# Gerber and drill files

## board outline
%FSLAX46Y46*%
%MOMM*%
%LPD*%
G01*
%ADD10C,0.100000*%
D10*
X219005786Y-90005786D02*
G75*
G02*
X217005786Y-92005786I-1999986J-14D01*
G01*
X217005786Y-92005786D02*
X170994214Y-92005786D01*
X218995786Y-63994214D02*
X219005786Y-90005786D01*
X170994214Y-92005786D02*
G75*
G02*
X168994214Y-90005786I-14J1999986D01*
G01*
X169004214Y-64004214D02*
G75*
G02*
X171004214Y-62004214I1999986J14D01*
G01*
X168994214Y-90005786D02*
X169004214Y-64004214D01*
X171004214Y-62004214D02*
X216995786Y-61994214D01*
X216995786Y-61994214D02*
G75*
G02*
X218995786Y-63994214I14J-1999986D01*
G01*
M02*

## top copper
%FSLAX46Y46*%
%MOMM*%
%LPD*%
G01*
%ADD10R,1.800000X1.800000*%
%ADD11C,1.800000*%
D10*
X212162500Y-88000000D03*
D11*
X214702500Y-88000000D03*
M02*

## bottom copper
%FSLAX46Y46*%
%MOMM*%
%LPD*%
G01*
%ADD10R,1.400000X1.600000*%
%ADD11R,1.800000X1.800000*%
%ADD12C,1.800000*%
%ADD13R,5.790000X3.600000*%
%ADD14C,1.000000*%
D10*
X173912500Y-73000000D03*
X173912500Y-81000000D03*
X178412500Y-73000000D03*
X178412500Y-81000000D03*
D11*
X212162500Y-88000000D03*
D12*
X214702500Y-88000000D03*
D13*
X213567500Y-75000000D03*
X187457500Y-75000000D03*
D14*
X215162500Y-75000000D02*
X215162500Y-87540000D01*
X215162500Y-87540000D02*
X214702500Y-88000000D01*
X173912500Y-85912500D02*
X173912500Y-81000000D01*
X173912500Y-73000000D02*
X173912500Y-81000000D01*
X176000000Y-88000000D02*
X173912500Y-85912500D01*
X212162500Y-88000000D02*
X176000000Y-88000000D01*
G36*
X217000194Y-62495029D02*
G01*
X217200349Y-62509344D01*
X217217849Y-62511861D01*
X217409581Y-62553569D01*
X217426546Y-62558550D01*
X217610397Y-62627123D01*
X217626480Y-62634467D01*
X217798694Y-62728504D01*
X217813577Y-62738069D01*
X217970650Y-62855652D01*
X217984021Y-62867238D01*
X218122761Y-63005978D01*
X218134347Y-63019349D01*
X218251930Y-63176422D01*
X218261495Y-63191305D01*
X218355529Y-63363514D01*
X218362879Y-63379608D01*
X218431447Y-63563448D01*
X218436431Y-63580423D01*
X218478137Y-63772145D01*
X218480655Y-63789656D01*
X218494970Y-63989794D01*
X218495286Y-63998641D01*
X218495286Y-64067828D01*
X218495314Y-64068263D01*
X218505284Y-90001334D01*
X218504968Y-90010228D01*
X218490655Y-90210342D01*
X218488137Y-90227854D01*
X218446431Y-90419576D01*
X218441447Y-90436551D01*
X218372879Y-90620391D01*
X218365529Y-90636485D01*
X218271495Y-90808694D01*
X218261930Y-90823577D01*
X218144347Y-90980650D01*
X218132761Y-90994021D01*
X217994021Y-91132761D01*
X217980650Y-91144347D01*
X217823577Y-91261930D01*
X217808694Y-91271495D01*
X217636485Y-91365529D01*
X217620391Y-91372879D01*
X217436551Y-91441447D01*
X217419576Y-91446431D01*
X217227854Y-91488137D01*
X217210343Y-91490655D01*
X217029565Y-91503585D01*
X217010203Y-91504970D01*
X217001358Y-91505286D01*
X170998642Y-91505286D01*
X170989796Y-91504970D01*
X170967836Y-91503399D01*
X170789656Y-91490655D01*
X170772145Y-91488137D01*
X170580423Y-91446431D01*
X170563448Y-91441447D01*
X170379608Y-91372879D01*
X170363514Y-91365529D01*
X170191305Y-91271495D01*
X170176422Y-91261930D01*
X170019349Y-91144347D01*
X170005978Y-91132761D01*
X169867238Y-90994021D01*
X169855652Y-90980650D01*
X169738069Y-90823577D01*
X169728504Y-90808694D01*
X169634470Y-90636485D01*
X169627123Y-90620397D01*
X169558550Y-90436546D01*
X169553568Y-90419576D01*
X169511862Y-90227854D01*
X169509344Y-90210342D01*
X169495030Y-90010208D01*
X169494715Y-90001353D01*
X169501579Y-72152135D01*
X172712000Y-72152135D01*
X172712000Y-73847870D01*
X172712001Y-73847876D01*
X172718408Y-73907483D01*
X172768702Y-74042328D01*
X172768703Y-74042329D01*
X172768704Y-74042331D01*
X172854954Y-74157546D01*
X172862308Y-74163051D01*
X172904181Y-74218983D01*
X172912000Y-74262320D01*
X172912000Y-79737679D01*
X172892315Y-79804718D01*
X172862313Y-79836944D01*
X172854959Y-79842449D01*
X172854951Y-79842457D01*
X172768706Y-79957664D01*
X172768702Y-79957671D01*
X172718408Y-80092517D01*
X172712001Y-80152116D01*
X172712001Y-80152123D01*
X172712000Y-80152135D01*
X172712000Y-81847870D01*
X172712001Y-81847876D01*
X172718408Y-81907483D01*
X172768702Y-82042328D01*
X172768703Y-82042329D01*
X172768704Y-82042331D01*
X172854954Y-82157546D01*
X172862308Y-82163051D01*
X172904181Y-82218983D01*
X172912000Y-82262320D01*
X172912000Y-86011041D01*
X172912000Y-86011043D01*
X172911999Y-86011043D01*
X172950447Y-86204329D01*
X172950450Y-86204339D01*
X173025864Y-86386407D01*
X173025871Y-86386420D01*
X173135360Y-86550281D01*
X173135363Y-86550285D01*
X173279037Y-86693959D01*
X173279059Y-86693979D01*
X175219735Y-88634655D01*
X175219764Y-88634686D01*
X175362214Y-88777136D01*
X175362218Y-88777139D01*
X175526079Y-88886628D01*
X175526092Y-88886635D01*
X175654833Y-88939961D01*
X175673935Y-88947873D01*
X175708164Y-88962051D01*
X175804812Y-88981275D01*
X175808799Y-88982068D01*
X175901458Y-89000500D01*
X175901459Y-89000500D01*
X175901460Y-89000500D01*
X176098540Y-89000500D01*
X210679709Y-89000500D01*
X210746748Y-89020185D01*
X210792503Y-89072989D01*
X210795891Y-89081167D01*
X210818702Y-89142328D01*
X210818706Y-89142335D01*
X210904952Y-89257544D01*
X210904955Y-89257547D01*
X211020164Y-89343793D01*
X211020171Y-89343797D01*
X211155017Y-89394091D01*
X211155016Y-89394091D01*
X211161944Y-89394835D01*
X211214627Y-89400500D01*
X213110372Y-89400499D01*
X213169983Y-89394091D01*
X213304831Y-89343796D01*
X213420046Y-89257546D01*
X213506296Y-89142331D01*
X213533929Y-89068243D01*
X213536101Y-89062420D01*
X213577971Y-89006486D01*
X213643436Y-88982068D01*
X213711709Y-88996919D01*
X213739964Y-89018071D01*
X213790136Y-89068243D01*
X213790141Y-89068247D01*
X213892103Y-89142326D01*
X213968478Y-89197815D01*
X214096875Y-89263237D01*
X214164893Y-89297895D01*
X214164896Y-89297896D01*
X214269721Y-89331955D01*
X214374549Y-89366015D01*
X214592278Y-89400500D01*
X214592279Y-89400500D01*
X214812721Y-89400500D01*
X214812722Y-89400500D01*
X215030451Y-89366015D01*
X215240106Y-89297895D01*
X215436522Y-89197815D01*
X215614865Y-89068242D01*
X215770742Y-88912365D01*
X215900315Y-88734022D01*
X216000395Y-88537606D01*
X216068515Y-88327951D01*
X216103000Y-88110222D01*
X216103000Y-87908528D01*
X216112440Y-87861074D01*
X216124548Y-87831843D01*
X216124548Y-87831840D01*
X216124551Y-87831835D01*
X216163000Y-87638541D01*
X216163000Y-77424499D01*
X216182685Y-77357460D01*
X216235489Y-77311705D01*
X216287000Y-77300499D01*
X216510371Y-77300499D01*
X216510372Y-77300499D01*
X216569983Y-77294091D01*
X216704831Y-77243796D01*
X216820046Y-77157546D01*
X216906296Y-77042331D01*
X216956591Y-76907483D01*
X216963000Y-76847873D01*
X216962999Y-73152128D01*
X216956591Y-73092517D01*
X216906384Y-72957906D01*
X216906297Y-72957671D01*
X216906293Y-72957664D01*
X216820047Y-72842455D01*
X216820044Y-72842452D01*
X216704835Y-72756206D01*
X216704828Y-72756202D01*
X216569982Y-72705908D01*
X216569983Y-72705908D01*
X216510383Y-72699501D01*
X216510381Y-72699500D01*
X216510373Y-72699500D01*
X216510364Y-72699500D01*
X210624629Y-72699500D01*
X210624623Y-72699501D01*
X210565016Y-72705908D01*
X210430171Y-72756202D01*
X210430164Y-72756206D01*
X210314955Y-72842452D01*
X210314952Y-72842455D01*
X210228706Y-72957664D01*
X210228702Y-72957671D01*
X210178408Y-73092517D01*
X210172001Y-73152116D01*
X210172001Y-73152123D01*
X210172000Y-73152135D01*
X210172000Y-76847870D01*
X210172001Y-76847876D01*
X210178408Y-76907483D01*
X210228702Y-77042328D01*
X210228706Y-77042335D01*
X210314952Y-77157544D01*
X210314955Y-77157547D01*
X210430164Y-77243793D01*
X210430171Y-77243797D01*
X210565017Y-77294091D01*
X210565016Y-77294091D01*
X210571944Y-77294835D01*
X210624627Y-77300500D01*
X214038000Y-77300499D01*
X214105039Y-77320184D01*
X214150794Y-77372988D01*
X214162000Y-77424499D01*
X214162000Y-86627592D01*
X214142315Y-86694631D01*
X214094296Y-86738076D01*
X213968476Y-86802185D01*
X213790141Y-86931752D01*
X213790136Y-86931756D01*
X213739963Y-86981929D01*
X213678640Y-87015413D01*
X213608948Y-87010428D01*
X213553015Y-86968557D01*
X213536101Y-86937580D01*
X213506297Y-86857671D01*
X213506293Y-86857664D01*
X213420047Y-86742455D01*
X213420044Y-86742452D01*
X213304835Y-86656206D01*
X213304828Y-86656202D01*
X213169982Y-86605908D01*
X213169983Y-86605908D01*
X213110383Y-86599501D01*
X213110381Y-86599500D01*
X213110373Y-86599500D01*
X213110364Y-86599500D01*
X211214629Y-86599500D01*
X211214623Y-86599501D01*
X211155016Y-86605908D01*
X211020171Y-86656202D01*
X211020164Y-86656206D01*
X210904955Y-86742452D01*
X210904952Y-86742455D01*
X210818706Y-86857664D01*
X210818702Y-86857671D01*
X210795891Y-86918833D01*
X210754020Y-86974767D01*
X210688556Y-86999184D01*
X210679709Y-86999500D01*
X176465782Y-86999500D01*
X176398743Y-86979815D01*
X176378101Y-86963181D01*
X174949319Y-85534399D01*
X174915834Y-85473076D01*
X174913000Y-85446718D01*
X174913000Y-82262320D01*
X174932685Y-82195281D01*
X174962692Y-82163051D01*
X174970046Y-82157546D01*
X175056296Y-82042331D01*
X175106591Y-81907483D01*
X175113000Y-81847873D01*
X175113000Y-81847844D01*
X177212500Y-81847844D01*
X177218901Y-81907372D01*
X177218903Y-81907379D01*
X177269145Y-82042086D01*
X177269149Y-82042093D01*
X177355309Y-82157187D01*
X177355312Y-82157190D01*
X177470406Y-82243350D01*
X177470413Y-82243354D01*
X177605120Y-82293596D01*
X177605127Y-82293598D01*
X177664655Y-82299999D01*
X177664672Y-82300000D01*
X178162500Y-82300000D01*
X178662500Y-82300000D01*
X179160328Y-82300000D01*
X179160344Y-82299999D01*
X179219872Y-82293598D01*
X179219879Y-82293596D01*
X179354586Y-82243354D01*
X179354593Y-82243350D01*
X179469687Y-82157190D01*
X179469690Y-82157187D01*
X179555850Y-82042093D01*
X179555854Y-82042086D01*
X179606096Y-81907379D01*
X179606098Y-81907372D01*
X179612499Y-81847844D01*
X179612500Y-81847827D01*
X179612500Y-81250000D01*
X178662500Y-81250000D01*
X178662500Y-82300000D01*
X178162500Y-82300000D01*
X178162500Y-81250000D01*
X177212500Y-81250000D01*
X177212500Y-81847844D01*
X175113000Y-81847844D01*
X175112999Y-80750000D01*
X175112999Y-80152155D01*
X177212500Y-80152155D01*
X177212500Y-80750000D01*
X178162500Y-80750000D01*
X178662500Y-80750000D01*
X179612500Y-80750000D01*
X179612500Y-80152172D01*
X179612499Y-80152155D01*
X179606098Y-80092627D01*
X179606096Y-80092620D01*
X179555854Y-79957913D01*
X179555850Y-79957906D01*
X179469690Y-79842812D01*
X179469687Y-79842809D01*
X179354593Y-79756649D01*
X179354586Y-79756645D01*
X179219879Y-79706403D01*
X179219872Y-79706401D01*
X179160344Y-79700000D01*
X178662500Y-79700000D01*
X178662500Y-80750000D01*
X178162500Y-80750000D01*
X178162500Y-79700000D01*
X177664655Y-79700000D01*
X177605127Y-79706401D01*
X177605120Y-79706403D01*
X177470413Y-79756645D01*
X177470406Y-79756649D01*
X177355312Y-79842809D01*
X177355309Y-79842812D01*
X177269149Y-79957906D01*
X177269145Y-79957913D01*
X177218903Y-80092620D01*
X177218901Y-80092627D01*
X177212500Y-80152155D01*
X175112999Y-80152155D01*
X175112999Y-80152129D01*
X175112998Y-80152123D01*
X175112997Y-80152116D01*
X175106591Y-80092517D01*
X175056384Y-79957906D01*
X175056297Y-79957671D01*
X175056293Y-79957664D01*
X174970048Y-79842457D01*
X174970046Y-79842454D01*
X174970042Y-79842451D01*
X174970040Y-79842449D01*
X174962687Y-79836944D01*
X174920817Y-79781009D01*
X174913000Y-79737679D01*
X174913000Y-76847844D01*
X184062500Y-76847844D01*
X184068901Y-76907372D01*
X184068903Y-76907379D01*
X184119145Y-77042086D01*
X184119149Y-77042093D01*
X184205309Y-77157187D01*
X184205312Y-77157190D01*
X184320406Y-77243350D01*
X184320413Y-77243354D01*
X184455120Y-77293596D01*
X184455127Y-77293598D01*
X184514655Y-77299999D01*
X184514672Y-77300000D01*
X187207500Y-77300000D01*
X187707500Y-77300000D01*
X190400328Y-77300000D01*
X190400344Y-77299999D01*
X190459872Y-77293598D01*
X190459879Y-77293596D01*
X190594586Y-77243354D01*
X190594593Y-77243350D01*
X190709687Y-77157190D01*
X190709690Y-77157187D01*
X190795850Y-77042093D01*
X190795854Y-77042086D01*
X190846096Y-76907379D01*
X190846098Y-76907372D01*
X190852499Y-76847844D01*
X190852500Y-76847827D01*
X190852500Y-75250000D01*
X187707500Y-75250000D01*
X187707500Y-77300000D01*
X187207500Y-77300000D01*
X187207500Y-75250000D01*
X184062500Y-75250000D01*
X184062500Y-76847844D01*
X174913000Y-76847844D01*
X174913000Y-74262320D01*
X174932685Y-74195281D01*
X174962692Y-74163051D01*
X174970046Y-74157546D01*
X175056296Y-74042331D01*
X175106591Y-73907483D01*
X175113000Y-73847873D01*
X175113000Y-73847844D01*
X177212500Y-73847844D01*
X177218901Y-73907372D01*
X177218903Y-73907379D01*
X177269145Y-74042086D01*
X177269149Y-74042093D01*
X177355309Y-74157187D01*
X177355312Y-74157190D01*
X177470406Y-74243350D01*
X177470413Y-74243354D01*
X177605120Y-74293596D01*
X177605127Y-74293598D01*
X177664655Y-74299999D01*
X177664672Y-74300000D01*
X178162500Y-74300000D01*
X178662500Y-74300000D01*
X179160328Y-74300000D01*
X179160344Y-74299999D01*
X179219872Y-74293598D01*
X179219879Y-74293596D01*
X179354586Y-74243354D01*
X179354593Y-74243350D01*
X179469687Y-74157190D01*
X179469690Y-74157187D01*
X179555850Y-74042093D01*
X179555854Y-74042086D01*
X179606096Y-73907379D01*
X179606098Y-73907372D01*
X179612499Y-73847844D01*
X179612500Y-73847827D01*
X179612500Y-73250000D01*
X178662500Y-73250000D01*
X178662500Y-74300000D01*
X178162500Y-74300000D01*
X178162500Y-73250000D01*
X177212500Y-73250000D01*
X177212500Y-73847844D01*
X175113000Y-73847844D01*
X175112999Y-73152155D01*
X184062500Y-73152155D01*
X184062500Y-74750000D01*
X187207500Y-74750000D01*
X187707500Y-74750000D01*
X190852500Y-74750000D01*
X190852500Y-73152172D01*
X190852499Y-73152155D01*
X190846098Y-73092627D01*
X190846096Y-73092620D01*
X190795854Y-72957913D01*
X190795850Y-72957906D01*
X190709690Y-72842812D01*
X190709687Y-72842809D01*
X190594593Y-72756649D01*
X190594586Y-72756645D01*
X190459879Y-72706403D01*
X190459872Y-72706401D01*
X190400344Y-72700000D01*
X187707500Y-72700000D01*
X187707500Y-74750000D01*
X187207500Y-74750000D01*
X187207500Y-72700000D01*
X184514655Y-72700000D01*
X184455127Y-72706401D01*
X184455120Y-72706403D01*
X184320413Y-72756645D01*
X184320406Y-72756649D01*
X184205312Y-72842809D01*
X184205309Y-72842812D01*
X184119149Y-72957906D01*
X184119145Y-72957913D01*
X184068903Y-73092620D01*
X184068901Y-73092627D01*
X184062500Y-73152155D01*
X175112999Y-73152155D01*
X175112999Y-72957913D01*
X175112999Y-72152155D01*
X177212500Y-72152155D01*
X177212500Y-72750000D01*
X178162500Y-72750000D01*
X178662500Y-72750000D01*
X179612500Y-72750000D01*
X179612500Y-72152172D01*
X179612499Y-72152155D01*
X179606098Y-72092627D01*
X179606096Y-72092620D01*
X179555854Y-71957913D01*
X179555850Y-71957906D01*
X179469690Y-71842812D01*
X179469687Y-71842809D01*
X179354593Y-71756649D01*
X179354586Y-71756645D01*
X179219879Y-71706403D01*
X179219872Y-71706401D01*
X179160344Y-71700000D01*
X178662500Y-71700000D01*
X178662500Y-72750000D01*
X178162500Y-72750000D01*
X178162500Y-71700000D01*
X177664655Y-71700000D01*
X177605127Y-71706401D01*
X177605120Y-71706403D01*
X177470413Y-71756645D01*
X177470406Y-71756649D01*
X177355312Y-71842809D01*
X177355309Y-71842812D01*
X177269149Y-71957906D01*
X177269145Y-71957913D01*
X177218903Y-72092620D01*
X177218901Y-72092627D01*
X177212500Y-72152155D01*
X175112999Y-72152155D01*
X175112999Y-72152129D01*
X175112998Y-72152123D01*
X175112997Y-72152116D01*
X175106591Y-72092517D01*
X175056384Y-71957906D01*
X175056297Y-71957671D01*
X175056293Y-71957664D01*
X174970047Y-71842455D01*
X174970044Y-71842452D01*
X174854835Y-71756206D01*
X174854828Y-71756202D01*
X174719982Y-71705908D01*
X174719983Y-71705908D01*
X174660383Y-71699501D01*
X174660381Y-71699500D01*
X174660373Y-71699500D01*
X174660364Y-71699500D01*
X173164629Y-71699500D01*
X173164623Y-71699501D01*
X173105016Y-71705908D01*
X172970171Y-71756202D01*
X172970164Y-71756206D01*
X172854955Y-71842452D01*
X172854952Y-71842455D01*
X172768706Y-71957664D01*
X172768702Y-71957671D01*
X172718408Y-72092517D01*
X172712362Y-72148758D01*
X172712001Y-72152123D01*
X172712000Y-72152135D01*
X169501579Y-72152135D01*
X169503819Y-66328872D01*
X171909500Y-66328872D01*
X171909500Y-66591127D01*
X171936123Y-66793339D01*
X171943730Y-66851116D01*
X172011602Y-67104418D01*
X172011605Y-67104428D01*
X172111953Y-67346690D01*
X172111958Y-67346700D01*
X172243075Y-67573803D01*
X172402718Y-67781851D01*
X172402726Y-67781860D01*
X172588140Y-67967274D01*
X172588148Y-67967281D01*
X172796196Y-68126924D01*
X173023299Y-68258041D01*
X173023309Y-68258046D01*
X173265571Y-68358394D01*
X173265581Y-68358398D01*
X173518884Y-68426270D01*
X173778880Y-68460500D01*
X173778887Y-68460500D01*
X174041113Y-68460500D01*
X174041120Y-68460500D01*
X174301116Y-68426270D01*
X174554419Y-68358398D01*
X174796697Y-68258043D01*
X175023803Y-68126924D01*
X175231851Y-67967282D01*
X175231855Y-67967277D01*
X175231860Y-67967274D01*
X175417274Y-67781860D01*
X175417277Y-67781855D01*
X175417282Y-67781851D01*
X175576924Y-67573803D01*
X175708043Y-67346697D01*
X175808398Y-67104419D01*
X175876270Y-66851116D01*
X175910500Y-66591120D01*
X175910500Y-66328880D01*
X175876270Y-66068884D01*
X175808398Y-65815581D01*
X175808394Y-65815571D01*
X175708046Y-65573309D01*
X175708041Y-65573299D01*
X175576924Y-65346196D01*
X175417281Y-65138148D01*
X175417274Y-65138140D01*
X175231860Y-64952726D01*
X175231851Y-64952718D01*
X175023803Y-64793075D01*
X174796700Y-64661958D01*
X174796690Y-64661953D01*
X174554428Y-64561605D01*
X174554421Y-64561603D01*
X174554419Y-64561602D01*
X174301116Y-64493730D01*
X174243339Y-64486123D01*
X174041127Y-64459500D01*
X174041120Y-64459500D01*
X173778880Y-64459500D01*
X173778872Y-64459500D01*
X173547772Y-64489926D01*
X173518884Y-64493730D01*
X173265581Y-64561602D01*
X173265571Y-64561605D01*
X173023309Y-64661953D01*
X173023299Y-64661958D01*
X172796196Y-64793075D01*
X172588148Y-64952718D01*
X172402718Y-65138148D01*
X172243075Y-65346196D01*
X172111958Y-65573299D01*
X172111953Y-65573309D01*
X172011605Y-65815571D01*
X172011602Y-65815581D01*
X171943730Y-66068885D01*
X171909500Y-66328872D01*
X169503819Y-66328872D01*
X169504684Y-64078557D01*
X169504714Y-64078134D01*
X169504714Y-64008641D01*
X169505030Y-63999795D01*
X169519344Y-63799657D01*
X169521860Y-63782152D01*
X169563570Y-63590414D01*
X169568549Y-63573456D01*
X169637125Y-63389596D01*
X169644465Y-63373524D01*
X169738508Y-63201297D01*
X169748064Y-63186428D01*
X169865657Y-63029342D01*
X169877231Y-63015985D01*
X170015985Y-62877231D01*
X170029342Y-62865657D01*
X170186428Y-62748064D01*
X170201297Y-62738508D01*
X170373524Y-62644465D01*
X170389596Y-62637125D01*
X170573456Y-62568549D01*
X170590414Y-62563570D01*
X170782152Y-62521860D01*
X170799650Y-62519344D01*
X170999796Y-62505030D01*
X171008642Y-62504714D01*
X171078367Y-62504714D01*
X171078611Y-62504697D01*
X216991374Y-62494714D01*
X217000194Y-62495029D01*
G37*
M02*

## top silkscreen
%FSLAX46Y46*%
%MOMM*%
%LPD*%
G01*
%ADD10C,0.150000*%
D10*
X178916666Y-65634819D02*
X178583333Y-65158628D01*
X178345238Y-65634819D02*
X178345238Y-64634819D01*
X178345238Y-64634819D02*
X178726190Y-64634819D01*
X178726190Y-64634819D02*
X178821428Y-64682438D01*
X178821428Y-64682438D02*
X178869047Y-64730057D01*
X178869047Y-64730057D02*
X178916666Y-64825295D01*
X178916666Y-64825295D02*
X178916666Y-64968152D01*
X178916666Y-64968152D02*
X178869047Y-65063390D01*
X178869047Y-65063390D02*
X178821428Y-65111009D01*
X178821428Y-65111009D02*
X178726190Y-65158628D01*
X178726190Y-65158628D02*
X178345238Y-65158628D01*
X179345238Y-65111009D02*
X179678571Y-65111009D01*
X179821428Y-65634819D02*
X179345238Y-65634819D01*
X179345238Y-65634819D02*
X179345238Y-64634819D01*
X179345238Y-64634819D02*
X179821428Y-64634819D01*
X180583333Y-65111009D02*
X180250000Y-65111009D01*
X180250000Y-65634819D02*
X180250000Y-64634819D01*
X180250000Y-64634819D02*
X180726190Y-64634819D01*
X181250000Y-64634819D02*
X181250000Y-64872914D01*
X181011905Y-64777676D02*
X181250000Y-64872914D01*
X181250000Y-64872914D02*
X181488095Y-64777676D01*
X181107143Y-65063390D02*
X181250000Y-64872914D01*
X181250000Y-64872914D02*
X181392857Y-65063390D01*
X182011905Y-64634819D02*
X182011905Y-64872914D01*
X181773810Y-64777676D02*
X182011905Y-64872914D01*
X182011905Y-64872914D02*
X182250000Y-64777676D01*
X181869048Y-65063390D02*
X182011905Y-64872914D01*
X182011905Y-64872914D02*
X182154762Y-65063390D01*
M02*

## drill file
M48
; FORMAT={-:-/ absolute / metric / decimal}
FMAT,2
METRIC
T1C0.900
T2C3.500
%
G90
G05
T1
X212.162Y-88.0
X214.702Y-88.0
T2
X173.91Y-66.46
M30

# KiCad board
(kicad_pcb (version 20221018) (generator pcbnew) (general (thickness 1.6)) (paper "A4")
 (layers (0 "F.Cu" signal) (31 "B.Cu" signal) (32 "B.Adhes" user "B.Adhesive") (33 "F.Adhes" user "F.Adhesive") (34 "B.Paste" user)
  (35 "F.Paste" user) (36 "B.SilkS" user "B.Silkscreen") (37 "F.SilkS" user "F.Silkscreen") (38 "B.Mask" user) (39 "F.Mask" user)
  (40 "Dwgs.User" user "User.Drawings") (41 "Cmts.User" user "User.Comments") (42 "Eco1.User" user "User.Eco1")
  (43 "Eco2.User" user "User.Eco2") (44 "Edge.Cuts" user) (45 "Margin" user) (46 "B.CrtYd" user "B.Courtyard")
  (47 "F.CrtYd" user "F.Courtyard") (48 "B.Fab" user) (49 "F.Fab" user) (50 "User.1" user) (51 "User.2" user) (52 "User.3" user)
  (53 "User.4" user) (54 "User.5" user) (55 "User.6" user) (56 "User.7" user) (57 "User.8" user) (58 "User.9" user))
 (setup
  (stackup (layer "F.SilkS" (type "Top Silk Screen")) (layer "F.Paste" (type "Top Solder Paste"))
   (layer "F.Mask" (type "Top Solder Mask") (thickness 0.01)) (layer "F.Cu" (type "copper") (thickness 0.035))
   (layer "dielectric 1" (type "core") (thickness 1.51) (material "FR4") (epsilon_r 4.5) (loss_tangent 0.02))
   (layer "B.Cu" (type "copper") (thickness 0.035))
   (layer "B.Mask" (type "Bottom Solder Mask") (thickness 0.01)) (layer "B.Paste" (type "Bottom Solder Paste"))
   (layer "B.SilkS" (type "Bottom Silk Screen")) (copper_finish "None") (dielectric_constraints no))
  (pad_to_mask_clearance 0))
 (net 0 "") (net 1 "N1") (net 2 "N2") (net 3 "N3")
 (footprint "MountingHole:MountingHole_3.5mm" (layer "F.Cu") (at 173.91 66.46)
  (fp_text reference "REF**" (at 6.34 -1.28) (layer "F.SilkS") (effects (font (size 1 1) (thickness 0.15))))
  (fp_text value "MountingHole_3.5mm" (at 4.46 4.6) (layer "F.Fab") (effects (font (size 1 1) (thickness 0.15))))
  (pad "" np_thru_hole circle (at 0 0) (size 3.5 3.5) (drill 3.5) (layers "*.Cu" "*.Mask")))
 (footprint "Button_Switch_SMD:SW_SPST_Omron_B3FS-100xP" (layer "B.Cu") (at 176.1625 77 -90)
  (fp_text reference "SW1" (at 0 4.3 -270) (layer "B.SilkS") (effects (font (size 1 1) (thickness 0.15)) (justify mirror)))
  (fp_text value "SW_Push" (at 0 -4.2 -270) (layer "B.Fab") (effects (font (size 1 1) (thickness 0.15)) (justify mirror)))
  (pad "1" smd rect (at -4 2.25 90) (size 1.6 1.4) (layers "B.Cu" "B.Paste" "B.Mask") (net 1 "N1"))
  (pad "1" smd rect (at 4 2.25 90) (size 1.6 1.4) (layers "B.Cu" "B.Paste" "B.Mask") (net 1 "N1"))
  (pad "2" smd rect (at -4 -2.25 90) (size 1.6 1.4) (layers "B.Cu" "B.Paste" "B.Mask") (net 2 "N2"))
  (pad "2" smd rect (at 4 -2.25 90) (size 1.6 1.4) (layers "B.Cu" "B.Paste" "B.Mask") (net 2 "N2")))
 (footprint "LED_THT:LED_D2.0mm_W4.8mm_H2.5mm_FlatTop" (layer "B.Cu") (at 212.1625 88)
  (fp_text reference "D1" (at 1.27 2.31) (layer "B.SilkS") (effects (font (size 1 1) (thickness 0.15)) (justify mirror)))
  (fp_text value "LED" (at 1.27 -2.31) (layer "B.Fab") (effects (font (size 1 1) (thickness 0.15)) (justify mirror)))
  (pad "1" thru_hole rect (at 0 0) (size 1.8 1.8) (drill 0.9) (layers "*.Cu" "*.Mask") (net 1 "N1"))
  (pad "2" thru_hole circle (at 2.54 0) (size 1.8 1.8) (drill 0.9) (layers "*.Cu" "*.Mask") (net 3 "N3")))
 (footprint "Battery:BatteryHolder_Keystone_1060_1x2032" (layer "B.Cu") (at 200.5125 75 180)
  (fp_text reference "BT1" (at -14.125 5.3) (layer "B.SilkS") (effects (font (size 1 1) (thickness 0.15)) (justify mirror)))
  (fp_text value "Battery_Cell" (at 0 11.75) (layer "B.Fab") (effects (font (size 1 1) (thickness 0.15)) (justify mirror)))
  (pad "1" smd rect (at -13.055 0) (size 5.79 3.6) (layers "B.Cu" "B.Paste" "B.Mask") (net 3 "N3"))
  (pad "2" smd rect (at 13.055 0) (size 5.79 3.6) (layers "B.Cu" "B.Paste" "B.Mask") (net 2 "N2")))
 (gr_arc (start 219.005786 90.005786) (mid 218.42 91.42) (end 217.005786 92.005786) (stroke (width 0.1) (type default)) (layer "Edge.Cuts"))
 (gr_line (start 217.005786 92.005786) (end 170.994214 92.005786) (stroke (width 0.1) (type default)) (layer "Edge.Cuts"))
 (gr_line (start 218.995786 63.994214) (end 219.005786 90.005786) (stroke (width 0.1) (type default)) (layer "Edge.Cuts"))
 (gr_arc (start 170.994214 92.005786) (mid 169.58 91.42) (end 168.994214 90.005786) (stroke (width 0.1) (type default)) (layer "Edge.Cuts"))
 (gr_arc (start 169.004214 64.004214) (mid 169.59 62.59) (end 171.004214 62.004214) (stroke (width 0.1) (type default)) (layer "Edge.Cuts"))
 (gr_line (start 168.994214 90.005786) (end 169.004214 64.004214) (stroke (width 0.1) (type default)) (layer "Edge.Cuts"))
 (gr_line (start 171.004214 62.004214) (end 216.995786 61.994214) (stroke (width 0.1) (type default)) (layer "Edge.Cuts"))
 (gr_arc (start 216.995786 61.994214) (mid 218.41 62.58) (end 218.995786 63.994214) (stroke (width 0.1) (type default)) (layer "Edge.Cuts"))
 (segment (start 215.1625 75) (end 215.1625 87.54) (width 1) (layer "B.Cu") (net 3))
 (segment (start 215.1625 87.54) (end 214.7025 88) (width 1) (layer "B.Cu") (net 3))
 (segment (start 173.9125 85.9125) (end 173.9125 81) (width 1) (layer "B.Cu") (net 1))
 (segment (start 173.9125 73) (end 173.9125 81) (width 1) (layer "B.Cu") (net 1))
 (segment (start 176 88) (end 173.9125 85.9125) (width 1) (layer "B.Cu") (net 1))
 (segment (start 212.1625 88) (end 176 88) (width 1) (layer "B.Cu") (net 1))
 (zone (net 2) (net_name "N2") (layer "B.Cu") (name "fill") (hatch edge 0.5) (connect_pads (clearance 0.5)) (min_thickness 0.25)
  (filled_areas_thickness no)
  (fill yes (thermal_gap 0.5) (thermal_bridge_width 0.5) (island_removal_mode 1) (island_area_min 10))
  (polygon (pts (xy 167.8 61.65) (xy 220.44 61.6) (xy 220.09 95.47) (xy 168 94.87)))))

